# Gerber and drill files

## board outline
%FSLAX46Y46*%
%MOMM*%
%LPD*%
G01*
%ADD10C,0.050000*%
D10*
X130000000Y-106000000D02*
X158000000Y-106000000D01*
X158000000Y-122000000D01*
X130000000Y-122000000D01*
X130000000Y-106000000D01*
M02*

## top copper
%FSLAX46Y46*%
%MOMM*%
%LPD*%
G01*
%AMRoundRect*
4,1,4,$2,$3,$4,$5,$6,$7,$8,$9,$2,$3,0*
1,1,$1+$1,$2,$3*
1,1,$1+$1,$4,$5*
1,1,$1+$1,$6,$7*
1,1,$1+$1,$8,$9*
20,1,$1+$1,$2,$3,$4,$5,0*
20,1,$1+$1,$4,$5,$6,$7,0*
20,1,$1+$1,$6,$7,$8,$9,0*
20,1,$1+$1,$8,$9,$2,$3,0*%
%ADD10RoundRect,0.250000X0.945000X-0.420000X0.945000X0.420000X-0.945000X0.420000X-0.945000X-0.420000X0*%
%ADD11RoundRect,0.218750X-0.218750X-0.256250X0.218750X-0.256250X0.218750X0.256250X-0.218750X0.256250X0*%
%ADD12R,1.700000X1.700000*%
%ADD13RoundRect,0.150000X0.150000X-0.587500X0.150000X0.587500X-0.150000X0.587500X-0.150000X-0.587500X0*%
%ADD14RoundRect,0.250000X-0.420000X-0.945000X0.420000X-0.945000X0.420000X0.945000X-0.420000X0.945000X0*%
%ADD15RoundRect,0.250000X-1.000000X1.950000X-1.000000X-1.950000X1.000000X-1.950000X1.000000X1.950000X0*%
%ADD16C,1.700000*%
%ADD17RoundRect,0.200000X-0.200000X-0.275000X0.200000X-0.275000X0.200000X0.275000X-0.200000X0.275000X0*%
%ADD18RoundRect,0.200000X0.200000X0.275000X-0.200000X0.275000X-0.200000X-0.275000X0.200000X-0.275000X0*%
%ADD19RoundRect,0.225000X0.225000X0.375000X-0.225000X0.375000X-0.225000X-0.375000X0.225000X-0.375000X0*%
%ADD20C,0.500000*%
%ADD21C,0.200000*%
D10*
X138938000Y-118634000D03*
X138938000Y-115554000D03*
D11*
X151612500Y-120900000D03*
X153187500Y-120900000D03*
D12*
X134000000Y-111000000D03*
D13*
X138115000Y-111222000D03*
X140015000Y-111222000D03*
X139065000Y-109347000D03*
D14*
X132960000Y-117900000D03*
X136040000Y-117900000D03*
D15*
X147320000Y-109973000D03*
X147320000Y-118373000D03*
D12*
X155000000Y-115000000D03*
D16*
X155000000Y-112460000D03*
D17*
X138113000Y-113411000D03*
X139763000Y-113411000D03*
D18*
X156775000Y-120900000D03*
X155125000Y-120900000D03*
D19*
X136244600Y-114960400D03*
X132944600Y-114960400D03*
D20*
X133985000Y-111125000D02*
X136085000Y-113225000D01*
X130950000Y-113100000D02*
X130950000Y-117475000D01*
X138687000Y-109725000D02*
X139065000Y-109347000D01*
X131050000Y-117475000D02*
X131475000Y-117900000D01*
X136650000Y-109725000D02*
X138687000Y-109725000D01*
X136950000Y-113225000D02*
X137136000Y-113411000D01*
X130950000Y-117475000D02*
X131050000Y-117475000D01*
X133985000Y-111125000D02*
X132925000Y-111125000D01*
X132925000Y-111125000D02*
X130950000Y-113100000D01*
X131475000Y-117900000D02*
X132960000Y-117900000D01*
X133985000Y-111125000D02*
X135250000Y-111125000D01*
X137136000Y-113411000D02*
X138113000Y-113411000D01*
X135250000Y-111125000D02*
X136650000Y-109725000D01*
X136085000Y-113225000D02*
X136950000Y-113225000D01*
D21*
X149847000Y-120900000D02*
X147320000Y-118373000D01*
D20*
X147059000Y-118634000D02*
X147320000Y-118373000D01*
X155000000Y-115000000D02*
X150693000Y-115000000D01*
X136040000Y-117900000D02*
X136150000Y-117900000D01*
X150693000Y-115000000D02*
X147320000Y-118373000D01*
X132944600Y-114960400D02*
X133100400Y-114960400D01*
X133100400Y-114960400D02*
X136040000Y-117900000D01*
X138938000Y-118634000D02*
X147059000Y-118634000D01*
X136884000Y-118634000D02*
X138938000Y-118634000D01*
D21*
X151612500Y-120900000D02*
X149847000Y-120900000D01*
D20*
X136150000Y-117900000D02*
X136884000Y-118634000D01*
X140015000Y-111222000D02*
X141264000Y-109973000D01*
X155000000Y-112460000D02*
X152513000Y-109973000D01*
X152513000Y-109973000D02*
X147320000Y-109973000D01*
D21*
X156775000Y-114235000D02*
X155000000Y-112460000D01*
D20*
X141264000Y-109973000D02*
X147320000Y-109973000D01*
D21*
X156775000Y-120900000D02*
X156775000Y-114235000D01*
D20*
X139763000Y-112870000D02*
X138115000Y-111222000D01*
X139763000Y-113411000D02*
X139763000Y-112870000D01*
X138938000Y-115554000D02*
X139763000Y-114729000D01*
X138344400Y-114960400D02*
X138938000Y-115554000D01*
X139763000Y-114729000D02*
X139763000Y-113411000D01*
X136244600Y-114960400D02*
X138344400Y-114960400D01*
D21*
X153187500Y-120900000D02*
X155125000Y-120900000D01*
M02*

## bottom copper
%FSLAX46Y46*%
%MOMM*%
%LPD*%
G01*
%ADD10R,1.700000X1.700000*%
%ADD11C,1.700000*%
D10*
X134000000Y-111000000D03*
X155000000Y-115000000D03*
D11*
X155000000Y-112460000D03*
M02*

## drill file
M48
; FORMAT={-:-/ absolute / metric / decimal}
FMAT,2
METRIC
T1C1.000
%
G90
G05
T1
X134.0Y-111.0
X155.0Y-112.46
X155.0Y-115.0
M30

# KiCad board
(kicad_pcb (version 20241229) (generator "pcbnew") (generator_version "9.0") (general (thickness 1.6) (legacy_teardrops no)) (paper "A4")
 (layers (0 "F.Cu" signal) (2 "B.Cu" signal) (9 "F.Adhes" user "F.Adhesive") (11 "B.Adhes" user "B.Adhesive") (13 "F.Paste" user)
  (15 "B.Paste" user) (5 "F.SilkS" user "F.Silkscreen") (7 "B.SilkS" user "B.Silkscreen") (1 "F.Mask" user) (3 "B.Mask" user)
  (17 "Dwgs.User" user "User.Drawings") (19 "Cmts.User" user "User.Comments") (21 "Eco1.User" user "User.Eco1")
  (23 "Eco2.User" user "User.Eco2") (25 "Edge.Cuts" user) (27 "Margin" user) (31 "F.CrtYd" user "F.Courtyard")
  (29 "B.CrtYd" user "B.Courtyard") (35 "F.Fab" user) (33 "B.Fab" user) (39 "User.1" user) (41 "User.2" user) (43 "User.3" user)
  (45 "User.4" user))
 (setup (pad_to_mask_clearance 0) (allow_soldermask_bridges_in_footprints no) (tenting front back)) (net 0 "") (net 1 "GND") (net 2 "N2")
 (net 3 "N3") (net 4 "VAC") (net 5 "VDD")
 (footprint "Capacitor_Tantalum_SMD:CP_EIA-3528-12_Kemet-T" (layer "F.Cu") (at 138.938 117.094 90)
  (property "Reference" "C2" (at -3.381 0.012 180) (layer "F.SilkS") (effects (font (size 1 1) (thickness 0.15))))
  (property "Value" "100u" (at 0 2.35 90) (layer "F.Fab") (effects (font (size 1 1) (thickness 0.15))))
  (pad "1" smd roundrect (at -1.54 0 90) (size 1.34 2.39) (layers "F.Cu" "F.Mask" "F.Paste") (roundrect_rratio 0.186567) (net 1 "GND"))
  (pad "2" smd roundrect (at 1.54 0 90) (size 1.34 2.39) (layers "F.Cu" "F.Mask" "F.Paste") (roundrect_rratio 0.186567) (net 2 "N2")))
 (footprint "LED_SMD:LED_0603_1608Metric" (layer "F.Cu") (at 152.4 120.9)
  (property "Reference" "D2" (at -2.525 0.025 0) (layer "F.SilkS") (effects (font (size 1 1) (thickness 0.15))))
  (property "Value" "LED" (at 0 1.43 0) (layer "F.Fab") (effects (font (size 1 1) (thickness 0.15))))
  (pad "1" smd roundrect (at -0.7875 0) (size 0.875 0.95) (layers "F.Cu" "F.Mask" "F.Paste") (roundrect_rratio 0.25) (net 1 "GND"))
  (pad "2" smd roundrect (at 0.7875 0) (size 0.875 0.95) (layers "F.Cu" "F.Mask" "F.Paste") (roundrect_rratio 0.25) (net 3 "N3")))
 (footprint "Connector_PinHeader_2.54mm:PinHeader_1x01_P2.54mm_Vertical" (layer "F.Cu") (at 134 111)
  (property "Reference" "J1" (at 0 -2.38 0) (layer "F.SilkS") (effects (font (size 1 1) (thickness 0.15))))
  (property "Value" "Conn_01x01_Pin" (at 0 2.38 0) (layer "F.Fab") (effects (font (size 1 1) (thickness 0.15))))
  (pad "1" thru_hole rect (at 0 0) (size 1.7 1.7) (drill 1) (layers "*.Cu" "*.Mask") (remove_unused_layers no) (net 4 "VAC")))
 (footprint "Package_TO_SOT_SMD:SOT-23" (layer "F.Cu") (at 139.065 110.2845 90)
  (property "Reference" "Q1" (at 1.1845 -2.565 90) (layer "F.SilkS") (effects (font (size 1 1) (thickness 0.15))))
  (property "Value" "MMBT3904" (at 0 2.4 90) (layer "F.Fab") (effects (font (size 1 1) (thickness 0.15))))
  (pad "1" smd roundrect (at -0.9375 -0.95 90) (size 1.475 0.6) (layers "F.Cu" "F.Mask" "F.Paste") (roundrect_rratio 0.25) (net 2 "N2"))
  (pad "2" smd roundrect (at -0.9375 0.95 90) (size 1.475 0.6) (layers "F.Cu" "F.Mask" "F.Paste") (roundrect_rratio 0.25) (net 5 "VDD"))
  (pad "3" smd roundrect (at 0.9375 0 90) (size 1.475 0.6) (layers "F.Cu" "F.Mask" "F.Paste") (roundrect_rratio 0.25) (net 4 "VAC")))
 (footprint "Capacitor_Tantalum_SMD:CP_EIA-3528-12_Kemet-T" (layer "F.Cu") (at 134.5 117.9)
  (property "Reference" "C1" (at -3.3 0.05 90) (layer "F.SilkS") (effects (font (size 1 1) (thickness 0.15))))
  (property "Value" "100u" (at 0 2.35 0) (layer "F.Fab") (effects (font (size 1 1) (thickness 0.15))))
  (pad "1" smd roundrect (at -1.54 0) (size 1.34 2.39) (layers "F.Cu" "F.Mask" "F.Paste") (roundrect_rratio 0.186567) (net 4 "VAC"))
  (pad "2" smd roundrect (at 1.54 0) (size 1.34 2.39) (layers "F.Cu" "F.Mask" "F.Paste") (roundrect_rratio 0.186567) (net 1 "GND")))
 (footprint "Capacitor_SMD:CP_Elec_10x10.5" (layer "F.Cu") (at 147.32 114.173 -90)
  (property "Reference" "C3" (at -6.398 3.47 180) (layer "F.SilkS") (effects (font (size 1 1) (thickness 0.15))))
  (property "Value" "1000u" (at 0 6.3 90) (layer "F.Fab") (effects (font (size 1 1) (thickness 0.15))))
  (pad "1" smd roundrect (at -4.2 0 270) (size 4.4 2.5) (layers "F.Cu" "F.Mask" "F.Paste") (roundrect_rratio 0.1) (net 5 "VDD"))
  (pad "2" smd roundrect (at 4.2 0 270) (size 4.4 2.5) (layers "F.Cu" "F.Mask" "F.Paste") (roundrect_rratio 0.1) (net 1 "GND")))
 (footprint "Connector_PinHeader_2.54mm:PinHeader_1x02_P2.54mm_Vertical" (layer "F.Cu") (at 155 115 180)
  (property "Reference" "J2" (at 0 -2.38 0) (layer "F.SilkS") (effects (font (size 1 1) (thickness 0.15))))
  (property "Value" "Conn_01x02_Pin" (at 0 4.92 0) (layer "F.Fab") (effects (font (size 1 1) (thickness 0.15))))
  (pad "1" thru_hole rect (at 0 0 180) (size 1.7 1.7) (drill 1) (layers "*.Cu" "*.Mask") (remove_unused_layers no) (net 1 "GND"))
  (pad "2" thru_hole circle (at 0 2.54 180) (size 1.7 1.7) (drill 1) (layers "*.Cu" "*.Mask") (remove_unused_layers no) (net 5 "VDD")))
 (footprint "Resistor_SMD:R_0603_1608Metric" (layer "F.Cu") (at 138.938 113.411)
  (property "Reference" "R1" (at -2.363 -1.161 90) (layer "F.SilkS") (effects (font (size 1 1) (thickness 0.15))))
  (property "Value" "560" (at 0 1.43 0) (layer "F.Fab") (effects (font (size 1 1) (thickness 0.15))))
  (pad "1" smd roundrect (at -0.825 0) (size 0.8 0.95) (layers "F.Cu" "F.Mask" "F.Paste") (roundrect_rratio 0.25) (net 4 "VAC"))
  (pad "2" smd roundrect (at 0.825 0) (size 0.8 0.95) (layers "F.Cu" "F.Mask" "F.Paste") (roundrect_rratio 0.25) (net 2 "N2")))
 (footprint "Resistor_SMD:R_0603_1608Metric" (layer "F.Cu") (at 155.95 120.9 180)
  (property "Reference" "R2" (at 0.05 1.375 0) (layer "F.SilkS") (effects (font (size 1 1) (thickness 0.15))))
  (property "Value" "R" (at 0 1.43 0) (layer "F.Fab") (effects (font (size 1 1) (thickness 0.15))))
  (pad "1" smd roundrect (at -0.825 0 180) (size 0.8 0.95) (layers "F.Cu" "F.Mask" "F.Paste") (roundrect_rratio 0.25) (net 5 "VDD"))
  (pad "2" smd roundrect (at 0.825 0 180) (size 0.8 0.95) (layers "F.Cu" "F.Mask" "F.Paste") (roundrect_rratio 0.25) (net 3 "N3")))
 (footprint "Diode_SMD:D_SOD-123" (layer "F.Cu") (at 134.5946 114.9604 180)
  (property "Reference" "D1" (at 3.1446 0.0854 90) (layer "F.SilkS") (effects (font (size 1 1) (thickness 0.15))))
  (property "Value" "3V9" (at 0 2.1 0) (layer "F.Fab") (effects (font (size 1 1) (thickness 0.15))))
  (pad "1" smd roundrect (at -1.65 0 180) (size 0.9 1.2) (layers "F.Cu" "F.Mask" "F.Paste") (roundrect_rratio 0.25) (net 2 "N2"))
  (pad "2" smd roundrect (at 1.65 0 180) (size 0.9 1.2) (layers "F.Cu" "F.Mask" "F.Paste") (roundrect_rratio 0.25) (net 1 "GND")))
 (gr_rect (start 130 106) (end 158 122) (stroke (width 0.05) (type solid)) (fill no) (layer "Edge.Cuts"))
 (segment (start 133.985 111.125) (end 136.085 113.225) (width 0.5) (layer "F.Cu") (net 4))
 (segment (start 130.95 113.1) (end 130.95 117.475) (width 0.5) (layer "F.Cu") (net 4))
 (segment (start 138.687 109.725) (end 139.065 109.347) (width 0.5) (layer "F.Cu") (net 4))
 (segment (start 131.05 117.475) (end 131.475 117.9) (width 0.5) (layer "F.Cu") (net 4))
 (segment (start 136.65 109.725) (end 138.687 109.725) (width 0.5) (layer "F.Cu") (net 4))
 (segment (start 136.95 113.225) (end 137.136 113.411) (width 0.5) (layer "F.Cu") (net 4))
 (segment (start 130.95 117.475) (end 131.05 117.475) (width 0.5) (layer "F.Cu") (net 4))
 (segment (start 133.985 111.125) (end 132.925 111.125) (width 0.5) (layer "F.Cu") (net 4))
 (segment (start 132.925 111.125) (end 130.95 113.1) (width 0.5) (layer "F.Cu") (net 4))
 (segment (start 131.475 117.9) (end 132.96 117.9) (width 0.5) (layer "F.Cu") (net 4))
 (segment (start 133.985 111.125) (end 135.25 111.125) (width 0.5) (layer "F.Cu") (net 4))
 (segment (start 137.136 113.411) (end 138.113 113.411) (width 0.5) (layer "F.Cu") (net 4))
 (segment (start 135.25 111.125) (end 136.65 109.725) (width 0.5) (layer "F.Cu") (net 4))
 (segment (start 136.085 113.225) (end 136.95 113.225) (width 0.5) (layer "F.Cu") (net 4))
 (segment (start 149.847 120.9) (end 147.32 118.373) (width 0.2) (layer "F.Cu") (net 1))
 (segment (start 147.059 118.634) (end 147.32 118.373) (width 0.5) (layer "F.Cu") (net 1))
 (segment (start 155 115) (end 150.693 115) (width 0.5) (layer "F.Cu") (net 1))
 (segment (start 136.04 117.9) (end 136.15 117.9) (width 0.5) (layer "F.Cu") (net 1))
 (segment (start 150.693 115) (end 147.32 118.373) (width 0.5) (layer "F.Cu") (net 1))
 (segment (start 132.9446 114.9604) (end 133.1004 114.9604) (width 0.5) (layer "F.Cu") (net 1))
 (segment (start 133.1004 114.9604) (end 136.04 117.9) (width 0.5) (layer "F.Cu") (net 1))
 (segment (start 138.938 118.634) (end 147.059 118.634) (width 0.5) (layer "F.Cu") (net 1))
 (segment (start 136.884 118.634) (end 138.938 118.634) (width 0.5) (layer "F.Cu") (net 1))
 (segment (start 151.6125 120.9) (end 149.847 120.9) (width 0.2) (layer "F.Cu") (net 1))
 (segment (start 136.15 117.9) (end 136.884 118.634) (width 0.5) (layer "F.Cu") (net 1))
 (segment (start 140.015 111.222) (end 141.264 109.973) (width 0.5) (layer "F.Cu") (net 5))
 (segment (start 155 112.46) (end 152.513 109.973) (width 0.5) (layer "F.Cu") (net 5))
 (segment (start 152.513 109.973) (end 147.32 109.973) (width 0.5) (layer "F.Cu") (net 5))
 (segment (start 156.775 114.235) (end 155 112.46) (width 0.2) (layer "F.Cu") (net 5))
 (segment (start 141.264 109.973) (end 147.32 109.973) (width 0.5) (layer "F.Cu") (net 5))
 (segment (start 156.775 120.9) (end 156.775 114.235) (width 0.2) (layer "F.Cu") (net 5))
 (segment (start 139.763 112.87) (end 138.115 111.222) (width 0.5) (layer "F.Cu") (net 2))
 (segment (start 139.763 113.411) (end 139.763 112.87) (width 0.5) (layer "F.Cu") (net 2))
 (segment (start 138.938 115.554) (end 139.763 114.729) (width 0.5) (layer "F.Cu") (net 2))
 (segment (start 138.3444 114.9604) (end 138.938 115.554) (width 0.5) (layer "F.Cu") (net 2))
 (segment (start 139.763 114.729) (end 139.763 113.411) (width 0.5) (layer "F.Cu") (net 2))
 (segment (start 136.2446 114.9604) (end 138.3444 114.9604) (width 0.5) (layer "F.Cu") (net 2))
 (segment (start 153.1875 120.9) (end 155.125 120.9) (width 0.2) (layer "F.Cu") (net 3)))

